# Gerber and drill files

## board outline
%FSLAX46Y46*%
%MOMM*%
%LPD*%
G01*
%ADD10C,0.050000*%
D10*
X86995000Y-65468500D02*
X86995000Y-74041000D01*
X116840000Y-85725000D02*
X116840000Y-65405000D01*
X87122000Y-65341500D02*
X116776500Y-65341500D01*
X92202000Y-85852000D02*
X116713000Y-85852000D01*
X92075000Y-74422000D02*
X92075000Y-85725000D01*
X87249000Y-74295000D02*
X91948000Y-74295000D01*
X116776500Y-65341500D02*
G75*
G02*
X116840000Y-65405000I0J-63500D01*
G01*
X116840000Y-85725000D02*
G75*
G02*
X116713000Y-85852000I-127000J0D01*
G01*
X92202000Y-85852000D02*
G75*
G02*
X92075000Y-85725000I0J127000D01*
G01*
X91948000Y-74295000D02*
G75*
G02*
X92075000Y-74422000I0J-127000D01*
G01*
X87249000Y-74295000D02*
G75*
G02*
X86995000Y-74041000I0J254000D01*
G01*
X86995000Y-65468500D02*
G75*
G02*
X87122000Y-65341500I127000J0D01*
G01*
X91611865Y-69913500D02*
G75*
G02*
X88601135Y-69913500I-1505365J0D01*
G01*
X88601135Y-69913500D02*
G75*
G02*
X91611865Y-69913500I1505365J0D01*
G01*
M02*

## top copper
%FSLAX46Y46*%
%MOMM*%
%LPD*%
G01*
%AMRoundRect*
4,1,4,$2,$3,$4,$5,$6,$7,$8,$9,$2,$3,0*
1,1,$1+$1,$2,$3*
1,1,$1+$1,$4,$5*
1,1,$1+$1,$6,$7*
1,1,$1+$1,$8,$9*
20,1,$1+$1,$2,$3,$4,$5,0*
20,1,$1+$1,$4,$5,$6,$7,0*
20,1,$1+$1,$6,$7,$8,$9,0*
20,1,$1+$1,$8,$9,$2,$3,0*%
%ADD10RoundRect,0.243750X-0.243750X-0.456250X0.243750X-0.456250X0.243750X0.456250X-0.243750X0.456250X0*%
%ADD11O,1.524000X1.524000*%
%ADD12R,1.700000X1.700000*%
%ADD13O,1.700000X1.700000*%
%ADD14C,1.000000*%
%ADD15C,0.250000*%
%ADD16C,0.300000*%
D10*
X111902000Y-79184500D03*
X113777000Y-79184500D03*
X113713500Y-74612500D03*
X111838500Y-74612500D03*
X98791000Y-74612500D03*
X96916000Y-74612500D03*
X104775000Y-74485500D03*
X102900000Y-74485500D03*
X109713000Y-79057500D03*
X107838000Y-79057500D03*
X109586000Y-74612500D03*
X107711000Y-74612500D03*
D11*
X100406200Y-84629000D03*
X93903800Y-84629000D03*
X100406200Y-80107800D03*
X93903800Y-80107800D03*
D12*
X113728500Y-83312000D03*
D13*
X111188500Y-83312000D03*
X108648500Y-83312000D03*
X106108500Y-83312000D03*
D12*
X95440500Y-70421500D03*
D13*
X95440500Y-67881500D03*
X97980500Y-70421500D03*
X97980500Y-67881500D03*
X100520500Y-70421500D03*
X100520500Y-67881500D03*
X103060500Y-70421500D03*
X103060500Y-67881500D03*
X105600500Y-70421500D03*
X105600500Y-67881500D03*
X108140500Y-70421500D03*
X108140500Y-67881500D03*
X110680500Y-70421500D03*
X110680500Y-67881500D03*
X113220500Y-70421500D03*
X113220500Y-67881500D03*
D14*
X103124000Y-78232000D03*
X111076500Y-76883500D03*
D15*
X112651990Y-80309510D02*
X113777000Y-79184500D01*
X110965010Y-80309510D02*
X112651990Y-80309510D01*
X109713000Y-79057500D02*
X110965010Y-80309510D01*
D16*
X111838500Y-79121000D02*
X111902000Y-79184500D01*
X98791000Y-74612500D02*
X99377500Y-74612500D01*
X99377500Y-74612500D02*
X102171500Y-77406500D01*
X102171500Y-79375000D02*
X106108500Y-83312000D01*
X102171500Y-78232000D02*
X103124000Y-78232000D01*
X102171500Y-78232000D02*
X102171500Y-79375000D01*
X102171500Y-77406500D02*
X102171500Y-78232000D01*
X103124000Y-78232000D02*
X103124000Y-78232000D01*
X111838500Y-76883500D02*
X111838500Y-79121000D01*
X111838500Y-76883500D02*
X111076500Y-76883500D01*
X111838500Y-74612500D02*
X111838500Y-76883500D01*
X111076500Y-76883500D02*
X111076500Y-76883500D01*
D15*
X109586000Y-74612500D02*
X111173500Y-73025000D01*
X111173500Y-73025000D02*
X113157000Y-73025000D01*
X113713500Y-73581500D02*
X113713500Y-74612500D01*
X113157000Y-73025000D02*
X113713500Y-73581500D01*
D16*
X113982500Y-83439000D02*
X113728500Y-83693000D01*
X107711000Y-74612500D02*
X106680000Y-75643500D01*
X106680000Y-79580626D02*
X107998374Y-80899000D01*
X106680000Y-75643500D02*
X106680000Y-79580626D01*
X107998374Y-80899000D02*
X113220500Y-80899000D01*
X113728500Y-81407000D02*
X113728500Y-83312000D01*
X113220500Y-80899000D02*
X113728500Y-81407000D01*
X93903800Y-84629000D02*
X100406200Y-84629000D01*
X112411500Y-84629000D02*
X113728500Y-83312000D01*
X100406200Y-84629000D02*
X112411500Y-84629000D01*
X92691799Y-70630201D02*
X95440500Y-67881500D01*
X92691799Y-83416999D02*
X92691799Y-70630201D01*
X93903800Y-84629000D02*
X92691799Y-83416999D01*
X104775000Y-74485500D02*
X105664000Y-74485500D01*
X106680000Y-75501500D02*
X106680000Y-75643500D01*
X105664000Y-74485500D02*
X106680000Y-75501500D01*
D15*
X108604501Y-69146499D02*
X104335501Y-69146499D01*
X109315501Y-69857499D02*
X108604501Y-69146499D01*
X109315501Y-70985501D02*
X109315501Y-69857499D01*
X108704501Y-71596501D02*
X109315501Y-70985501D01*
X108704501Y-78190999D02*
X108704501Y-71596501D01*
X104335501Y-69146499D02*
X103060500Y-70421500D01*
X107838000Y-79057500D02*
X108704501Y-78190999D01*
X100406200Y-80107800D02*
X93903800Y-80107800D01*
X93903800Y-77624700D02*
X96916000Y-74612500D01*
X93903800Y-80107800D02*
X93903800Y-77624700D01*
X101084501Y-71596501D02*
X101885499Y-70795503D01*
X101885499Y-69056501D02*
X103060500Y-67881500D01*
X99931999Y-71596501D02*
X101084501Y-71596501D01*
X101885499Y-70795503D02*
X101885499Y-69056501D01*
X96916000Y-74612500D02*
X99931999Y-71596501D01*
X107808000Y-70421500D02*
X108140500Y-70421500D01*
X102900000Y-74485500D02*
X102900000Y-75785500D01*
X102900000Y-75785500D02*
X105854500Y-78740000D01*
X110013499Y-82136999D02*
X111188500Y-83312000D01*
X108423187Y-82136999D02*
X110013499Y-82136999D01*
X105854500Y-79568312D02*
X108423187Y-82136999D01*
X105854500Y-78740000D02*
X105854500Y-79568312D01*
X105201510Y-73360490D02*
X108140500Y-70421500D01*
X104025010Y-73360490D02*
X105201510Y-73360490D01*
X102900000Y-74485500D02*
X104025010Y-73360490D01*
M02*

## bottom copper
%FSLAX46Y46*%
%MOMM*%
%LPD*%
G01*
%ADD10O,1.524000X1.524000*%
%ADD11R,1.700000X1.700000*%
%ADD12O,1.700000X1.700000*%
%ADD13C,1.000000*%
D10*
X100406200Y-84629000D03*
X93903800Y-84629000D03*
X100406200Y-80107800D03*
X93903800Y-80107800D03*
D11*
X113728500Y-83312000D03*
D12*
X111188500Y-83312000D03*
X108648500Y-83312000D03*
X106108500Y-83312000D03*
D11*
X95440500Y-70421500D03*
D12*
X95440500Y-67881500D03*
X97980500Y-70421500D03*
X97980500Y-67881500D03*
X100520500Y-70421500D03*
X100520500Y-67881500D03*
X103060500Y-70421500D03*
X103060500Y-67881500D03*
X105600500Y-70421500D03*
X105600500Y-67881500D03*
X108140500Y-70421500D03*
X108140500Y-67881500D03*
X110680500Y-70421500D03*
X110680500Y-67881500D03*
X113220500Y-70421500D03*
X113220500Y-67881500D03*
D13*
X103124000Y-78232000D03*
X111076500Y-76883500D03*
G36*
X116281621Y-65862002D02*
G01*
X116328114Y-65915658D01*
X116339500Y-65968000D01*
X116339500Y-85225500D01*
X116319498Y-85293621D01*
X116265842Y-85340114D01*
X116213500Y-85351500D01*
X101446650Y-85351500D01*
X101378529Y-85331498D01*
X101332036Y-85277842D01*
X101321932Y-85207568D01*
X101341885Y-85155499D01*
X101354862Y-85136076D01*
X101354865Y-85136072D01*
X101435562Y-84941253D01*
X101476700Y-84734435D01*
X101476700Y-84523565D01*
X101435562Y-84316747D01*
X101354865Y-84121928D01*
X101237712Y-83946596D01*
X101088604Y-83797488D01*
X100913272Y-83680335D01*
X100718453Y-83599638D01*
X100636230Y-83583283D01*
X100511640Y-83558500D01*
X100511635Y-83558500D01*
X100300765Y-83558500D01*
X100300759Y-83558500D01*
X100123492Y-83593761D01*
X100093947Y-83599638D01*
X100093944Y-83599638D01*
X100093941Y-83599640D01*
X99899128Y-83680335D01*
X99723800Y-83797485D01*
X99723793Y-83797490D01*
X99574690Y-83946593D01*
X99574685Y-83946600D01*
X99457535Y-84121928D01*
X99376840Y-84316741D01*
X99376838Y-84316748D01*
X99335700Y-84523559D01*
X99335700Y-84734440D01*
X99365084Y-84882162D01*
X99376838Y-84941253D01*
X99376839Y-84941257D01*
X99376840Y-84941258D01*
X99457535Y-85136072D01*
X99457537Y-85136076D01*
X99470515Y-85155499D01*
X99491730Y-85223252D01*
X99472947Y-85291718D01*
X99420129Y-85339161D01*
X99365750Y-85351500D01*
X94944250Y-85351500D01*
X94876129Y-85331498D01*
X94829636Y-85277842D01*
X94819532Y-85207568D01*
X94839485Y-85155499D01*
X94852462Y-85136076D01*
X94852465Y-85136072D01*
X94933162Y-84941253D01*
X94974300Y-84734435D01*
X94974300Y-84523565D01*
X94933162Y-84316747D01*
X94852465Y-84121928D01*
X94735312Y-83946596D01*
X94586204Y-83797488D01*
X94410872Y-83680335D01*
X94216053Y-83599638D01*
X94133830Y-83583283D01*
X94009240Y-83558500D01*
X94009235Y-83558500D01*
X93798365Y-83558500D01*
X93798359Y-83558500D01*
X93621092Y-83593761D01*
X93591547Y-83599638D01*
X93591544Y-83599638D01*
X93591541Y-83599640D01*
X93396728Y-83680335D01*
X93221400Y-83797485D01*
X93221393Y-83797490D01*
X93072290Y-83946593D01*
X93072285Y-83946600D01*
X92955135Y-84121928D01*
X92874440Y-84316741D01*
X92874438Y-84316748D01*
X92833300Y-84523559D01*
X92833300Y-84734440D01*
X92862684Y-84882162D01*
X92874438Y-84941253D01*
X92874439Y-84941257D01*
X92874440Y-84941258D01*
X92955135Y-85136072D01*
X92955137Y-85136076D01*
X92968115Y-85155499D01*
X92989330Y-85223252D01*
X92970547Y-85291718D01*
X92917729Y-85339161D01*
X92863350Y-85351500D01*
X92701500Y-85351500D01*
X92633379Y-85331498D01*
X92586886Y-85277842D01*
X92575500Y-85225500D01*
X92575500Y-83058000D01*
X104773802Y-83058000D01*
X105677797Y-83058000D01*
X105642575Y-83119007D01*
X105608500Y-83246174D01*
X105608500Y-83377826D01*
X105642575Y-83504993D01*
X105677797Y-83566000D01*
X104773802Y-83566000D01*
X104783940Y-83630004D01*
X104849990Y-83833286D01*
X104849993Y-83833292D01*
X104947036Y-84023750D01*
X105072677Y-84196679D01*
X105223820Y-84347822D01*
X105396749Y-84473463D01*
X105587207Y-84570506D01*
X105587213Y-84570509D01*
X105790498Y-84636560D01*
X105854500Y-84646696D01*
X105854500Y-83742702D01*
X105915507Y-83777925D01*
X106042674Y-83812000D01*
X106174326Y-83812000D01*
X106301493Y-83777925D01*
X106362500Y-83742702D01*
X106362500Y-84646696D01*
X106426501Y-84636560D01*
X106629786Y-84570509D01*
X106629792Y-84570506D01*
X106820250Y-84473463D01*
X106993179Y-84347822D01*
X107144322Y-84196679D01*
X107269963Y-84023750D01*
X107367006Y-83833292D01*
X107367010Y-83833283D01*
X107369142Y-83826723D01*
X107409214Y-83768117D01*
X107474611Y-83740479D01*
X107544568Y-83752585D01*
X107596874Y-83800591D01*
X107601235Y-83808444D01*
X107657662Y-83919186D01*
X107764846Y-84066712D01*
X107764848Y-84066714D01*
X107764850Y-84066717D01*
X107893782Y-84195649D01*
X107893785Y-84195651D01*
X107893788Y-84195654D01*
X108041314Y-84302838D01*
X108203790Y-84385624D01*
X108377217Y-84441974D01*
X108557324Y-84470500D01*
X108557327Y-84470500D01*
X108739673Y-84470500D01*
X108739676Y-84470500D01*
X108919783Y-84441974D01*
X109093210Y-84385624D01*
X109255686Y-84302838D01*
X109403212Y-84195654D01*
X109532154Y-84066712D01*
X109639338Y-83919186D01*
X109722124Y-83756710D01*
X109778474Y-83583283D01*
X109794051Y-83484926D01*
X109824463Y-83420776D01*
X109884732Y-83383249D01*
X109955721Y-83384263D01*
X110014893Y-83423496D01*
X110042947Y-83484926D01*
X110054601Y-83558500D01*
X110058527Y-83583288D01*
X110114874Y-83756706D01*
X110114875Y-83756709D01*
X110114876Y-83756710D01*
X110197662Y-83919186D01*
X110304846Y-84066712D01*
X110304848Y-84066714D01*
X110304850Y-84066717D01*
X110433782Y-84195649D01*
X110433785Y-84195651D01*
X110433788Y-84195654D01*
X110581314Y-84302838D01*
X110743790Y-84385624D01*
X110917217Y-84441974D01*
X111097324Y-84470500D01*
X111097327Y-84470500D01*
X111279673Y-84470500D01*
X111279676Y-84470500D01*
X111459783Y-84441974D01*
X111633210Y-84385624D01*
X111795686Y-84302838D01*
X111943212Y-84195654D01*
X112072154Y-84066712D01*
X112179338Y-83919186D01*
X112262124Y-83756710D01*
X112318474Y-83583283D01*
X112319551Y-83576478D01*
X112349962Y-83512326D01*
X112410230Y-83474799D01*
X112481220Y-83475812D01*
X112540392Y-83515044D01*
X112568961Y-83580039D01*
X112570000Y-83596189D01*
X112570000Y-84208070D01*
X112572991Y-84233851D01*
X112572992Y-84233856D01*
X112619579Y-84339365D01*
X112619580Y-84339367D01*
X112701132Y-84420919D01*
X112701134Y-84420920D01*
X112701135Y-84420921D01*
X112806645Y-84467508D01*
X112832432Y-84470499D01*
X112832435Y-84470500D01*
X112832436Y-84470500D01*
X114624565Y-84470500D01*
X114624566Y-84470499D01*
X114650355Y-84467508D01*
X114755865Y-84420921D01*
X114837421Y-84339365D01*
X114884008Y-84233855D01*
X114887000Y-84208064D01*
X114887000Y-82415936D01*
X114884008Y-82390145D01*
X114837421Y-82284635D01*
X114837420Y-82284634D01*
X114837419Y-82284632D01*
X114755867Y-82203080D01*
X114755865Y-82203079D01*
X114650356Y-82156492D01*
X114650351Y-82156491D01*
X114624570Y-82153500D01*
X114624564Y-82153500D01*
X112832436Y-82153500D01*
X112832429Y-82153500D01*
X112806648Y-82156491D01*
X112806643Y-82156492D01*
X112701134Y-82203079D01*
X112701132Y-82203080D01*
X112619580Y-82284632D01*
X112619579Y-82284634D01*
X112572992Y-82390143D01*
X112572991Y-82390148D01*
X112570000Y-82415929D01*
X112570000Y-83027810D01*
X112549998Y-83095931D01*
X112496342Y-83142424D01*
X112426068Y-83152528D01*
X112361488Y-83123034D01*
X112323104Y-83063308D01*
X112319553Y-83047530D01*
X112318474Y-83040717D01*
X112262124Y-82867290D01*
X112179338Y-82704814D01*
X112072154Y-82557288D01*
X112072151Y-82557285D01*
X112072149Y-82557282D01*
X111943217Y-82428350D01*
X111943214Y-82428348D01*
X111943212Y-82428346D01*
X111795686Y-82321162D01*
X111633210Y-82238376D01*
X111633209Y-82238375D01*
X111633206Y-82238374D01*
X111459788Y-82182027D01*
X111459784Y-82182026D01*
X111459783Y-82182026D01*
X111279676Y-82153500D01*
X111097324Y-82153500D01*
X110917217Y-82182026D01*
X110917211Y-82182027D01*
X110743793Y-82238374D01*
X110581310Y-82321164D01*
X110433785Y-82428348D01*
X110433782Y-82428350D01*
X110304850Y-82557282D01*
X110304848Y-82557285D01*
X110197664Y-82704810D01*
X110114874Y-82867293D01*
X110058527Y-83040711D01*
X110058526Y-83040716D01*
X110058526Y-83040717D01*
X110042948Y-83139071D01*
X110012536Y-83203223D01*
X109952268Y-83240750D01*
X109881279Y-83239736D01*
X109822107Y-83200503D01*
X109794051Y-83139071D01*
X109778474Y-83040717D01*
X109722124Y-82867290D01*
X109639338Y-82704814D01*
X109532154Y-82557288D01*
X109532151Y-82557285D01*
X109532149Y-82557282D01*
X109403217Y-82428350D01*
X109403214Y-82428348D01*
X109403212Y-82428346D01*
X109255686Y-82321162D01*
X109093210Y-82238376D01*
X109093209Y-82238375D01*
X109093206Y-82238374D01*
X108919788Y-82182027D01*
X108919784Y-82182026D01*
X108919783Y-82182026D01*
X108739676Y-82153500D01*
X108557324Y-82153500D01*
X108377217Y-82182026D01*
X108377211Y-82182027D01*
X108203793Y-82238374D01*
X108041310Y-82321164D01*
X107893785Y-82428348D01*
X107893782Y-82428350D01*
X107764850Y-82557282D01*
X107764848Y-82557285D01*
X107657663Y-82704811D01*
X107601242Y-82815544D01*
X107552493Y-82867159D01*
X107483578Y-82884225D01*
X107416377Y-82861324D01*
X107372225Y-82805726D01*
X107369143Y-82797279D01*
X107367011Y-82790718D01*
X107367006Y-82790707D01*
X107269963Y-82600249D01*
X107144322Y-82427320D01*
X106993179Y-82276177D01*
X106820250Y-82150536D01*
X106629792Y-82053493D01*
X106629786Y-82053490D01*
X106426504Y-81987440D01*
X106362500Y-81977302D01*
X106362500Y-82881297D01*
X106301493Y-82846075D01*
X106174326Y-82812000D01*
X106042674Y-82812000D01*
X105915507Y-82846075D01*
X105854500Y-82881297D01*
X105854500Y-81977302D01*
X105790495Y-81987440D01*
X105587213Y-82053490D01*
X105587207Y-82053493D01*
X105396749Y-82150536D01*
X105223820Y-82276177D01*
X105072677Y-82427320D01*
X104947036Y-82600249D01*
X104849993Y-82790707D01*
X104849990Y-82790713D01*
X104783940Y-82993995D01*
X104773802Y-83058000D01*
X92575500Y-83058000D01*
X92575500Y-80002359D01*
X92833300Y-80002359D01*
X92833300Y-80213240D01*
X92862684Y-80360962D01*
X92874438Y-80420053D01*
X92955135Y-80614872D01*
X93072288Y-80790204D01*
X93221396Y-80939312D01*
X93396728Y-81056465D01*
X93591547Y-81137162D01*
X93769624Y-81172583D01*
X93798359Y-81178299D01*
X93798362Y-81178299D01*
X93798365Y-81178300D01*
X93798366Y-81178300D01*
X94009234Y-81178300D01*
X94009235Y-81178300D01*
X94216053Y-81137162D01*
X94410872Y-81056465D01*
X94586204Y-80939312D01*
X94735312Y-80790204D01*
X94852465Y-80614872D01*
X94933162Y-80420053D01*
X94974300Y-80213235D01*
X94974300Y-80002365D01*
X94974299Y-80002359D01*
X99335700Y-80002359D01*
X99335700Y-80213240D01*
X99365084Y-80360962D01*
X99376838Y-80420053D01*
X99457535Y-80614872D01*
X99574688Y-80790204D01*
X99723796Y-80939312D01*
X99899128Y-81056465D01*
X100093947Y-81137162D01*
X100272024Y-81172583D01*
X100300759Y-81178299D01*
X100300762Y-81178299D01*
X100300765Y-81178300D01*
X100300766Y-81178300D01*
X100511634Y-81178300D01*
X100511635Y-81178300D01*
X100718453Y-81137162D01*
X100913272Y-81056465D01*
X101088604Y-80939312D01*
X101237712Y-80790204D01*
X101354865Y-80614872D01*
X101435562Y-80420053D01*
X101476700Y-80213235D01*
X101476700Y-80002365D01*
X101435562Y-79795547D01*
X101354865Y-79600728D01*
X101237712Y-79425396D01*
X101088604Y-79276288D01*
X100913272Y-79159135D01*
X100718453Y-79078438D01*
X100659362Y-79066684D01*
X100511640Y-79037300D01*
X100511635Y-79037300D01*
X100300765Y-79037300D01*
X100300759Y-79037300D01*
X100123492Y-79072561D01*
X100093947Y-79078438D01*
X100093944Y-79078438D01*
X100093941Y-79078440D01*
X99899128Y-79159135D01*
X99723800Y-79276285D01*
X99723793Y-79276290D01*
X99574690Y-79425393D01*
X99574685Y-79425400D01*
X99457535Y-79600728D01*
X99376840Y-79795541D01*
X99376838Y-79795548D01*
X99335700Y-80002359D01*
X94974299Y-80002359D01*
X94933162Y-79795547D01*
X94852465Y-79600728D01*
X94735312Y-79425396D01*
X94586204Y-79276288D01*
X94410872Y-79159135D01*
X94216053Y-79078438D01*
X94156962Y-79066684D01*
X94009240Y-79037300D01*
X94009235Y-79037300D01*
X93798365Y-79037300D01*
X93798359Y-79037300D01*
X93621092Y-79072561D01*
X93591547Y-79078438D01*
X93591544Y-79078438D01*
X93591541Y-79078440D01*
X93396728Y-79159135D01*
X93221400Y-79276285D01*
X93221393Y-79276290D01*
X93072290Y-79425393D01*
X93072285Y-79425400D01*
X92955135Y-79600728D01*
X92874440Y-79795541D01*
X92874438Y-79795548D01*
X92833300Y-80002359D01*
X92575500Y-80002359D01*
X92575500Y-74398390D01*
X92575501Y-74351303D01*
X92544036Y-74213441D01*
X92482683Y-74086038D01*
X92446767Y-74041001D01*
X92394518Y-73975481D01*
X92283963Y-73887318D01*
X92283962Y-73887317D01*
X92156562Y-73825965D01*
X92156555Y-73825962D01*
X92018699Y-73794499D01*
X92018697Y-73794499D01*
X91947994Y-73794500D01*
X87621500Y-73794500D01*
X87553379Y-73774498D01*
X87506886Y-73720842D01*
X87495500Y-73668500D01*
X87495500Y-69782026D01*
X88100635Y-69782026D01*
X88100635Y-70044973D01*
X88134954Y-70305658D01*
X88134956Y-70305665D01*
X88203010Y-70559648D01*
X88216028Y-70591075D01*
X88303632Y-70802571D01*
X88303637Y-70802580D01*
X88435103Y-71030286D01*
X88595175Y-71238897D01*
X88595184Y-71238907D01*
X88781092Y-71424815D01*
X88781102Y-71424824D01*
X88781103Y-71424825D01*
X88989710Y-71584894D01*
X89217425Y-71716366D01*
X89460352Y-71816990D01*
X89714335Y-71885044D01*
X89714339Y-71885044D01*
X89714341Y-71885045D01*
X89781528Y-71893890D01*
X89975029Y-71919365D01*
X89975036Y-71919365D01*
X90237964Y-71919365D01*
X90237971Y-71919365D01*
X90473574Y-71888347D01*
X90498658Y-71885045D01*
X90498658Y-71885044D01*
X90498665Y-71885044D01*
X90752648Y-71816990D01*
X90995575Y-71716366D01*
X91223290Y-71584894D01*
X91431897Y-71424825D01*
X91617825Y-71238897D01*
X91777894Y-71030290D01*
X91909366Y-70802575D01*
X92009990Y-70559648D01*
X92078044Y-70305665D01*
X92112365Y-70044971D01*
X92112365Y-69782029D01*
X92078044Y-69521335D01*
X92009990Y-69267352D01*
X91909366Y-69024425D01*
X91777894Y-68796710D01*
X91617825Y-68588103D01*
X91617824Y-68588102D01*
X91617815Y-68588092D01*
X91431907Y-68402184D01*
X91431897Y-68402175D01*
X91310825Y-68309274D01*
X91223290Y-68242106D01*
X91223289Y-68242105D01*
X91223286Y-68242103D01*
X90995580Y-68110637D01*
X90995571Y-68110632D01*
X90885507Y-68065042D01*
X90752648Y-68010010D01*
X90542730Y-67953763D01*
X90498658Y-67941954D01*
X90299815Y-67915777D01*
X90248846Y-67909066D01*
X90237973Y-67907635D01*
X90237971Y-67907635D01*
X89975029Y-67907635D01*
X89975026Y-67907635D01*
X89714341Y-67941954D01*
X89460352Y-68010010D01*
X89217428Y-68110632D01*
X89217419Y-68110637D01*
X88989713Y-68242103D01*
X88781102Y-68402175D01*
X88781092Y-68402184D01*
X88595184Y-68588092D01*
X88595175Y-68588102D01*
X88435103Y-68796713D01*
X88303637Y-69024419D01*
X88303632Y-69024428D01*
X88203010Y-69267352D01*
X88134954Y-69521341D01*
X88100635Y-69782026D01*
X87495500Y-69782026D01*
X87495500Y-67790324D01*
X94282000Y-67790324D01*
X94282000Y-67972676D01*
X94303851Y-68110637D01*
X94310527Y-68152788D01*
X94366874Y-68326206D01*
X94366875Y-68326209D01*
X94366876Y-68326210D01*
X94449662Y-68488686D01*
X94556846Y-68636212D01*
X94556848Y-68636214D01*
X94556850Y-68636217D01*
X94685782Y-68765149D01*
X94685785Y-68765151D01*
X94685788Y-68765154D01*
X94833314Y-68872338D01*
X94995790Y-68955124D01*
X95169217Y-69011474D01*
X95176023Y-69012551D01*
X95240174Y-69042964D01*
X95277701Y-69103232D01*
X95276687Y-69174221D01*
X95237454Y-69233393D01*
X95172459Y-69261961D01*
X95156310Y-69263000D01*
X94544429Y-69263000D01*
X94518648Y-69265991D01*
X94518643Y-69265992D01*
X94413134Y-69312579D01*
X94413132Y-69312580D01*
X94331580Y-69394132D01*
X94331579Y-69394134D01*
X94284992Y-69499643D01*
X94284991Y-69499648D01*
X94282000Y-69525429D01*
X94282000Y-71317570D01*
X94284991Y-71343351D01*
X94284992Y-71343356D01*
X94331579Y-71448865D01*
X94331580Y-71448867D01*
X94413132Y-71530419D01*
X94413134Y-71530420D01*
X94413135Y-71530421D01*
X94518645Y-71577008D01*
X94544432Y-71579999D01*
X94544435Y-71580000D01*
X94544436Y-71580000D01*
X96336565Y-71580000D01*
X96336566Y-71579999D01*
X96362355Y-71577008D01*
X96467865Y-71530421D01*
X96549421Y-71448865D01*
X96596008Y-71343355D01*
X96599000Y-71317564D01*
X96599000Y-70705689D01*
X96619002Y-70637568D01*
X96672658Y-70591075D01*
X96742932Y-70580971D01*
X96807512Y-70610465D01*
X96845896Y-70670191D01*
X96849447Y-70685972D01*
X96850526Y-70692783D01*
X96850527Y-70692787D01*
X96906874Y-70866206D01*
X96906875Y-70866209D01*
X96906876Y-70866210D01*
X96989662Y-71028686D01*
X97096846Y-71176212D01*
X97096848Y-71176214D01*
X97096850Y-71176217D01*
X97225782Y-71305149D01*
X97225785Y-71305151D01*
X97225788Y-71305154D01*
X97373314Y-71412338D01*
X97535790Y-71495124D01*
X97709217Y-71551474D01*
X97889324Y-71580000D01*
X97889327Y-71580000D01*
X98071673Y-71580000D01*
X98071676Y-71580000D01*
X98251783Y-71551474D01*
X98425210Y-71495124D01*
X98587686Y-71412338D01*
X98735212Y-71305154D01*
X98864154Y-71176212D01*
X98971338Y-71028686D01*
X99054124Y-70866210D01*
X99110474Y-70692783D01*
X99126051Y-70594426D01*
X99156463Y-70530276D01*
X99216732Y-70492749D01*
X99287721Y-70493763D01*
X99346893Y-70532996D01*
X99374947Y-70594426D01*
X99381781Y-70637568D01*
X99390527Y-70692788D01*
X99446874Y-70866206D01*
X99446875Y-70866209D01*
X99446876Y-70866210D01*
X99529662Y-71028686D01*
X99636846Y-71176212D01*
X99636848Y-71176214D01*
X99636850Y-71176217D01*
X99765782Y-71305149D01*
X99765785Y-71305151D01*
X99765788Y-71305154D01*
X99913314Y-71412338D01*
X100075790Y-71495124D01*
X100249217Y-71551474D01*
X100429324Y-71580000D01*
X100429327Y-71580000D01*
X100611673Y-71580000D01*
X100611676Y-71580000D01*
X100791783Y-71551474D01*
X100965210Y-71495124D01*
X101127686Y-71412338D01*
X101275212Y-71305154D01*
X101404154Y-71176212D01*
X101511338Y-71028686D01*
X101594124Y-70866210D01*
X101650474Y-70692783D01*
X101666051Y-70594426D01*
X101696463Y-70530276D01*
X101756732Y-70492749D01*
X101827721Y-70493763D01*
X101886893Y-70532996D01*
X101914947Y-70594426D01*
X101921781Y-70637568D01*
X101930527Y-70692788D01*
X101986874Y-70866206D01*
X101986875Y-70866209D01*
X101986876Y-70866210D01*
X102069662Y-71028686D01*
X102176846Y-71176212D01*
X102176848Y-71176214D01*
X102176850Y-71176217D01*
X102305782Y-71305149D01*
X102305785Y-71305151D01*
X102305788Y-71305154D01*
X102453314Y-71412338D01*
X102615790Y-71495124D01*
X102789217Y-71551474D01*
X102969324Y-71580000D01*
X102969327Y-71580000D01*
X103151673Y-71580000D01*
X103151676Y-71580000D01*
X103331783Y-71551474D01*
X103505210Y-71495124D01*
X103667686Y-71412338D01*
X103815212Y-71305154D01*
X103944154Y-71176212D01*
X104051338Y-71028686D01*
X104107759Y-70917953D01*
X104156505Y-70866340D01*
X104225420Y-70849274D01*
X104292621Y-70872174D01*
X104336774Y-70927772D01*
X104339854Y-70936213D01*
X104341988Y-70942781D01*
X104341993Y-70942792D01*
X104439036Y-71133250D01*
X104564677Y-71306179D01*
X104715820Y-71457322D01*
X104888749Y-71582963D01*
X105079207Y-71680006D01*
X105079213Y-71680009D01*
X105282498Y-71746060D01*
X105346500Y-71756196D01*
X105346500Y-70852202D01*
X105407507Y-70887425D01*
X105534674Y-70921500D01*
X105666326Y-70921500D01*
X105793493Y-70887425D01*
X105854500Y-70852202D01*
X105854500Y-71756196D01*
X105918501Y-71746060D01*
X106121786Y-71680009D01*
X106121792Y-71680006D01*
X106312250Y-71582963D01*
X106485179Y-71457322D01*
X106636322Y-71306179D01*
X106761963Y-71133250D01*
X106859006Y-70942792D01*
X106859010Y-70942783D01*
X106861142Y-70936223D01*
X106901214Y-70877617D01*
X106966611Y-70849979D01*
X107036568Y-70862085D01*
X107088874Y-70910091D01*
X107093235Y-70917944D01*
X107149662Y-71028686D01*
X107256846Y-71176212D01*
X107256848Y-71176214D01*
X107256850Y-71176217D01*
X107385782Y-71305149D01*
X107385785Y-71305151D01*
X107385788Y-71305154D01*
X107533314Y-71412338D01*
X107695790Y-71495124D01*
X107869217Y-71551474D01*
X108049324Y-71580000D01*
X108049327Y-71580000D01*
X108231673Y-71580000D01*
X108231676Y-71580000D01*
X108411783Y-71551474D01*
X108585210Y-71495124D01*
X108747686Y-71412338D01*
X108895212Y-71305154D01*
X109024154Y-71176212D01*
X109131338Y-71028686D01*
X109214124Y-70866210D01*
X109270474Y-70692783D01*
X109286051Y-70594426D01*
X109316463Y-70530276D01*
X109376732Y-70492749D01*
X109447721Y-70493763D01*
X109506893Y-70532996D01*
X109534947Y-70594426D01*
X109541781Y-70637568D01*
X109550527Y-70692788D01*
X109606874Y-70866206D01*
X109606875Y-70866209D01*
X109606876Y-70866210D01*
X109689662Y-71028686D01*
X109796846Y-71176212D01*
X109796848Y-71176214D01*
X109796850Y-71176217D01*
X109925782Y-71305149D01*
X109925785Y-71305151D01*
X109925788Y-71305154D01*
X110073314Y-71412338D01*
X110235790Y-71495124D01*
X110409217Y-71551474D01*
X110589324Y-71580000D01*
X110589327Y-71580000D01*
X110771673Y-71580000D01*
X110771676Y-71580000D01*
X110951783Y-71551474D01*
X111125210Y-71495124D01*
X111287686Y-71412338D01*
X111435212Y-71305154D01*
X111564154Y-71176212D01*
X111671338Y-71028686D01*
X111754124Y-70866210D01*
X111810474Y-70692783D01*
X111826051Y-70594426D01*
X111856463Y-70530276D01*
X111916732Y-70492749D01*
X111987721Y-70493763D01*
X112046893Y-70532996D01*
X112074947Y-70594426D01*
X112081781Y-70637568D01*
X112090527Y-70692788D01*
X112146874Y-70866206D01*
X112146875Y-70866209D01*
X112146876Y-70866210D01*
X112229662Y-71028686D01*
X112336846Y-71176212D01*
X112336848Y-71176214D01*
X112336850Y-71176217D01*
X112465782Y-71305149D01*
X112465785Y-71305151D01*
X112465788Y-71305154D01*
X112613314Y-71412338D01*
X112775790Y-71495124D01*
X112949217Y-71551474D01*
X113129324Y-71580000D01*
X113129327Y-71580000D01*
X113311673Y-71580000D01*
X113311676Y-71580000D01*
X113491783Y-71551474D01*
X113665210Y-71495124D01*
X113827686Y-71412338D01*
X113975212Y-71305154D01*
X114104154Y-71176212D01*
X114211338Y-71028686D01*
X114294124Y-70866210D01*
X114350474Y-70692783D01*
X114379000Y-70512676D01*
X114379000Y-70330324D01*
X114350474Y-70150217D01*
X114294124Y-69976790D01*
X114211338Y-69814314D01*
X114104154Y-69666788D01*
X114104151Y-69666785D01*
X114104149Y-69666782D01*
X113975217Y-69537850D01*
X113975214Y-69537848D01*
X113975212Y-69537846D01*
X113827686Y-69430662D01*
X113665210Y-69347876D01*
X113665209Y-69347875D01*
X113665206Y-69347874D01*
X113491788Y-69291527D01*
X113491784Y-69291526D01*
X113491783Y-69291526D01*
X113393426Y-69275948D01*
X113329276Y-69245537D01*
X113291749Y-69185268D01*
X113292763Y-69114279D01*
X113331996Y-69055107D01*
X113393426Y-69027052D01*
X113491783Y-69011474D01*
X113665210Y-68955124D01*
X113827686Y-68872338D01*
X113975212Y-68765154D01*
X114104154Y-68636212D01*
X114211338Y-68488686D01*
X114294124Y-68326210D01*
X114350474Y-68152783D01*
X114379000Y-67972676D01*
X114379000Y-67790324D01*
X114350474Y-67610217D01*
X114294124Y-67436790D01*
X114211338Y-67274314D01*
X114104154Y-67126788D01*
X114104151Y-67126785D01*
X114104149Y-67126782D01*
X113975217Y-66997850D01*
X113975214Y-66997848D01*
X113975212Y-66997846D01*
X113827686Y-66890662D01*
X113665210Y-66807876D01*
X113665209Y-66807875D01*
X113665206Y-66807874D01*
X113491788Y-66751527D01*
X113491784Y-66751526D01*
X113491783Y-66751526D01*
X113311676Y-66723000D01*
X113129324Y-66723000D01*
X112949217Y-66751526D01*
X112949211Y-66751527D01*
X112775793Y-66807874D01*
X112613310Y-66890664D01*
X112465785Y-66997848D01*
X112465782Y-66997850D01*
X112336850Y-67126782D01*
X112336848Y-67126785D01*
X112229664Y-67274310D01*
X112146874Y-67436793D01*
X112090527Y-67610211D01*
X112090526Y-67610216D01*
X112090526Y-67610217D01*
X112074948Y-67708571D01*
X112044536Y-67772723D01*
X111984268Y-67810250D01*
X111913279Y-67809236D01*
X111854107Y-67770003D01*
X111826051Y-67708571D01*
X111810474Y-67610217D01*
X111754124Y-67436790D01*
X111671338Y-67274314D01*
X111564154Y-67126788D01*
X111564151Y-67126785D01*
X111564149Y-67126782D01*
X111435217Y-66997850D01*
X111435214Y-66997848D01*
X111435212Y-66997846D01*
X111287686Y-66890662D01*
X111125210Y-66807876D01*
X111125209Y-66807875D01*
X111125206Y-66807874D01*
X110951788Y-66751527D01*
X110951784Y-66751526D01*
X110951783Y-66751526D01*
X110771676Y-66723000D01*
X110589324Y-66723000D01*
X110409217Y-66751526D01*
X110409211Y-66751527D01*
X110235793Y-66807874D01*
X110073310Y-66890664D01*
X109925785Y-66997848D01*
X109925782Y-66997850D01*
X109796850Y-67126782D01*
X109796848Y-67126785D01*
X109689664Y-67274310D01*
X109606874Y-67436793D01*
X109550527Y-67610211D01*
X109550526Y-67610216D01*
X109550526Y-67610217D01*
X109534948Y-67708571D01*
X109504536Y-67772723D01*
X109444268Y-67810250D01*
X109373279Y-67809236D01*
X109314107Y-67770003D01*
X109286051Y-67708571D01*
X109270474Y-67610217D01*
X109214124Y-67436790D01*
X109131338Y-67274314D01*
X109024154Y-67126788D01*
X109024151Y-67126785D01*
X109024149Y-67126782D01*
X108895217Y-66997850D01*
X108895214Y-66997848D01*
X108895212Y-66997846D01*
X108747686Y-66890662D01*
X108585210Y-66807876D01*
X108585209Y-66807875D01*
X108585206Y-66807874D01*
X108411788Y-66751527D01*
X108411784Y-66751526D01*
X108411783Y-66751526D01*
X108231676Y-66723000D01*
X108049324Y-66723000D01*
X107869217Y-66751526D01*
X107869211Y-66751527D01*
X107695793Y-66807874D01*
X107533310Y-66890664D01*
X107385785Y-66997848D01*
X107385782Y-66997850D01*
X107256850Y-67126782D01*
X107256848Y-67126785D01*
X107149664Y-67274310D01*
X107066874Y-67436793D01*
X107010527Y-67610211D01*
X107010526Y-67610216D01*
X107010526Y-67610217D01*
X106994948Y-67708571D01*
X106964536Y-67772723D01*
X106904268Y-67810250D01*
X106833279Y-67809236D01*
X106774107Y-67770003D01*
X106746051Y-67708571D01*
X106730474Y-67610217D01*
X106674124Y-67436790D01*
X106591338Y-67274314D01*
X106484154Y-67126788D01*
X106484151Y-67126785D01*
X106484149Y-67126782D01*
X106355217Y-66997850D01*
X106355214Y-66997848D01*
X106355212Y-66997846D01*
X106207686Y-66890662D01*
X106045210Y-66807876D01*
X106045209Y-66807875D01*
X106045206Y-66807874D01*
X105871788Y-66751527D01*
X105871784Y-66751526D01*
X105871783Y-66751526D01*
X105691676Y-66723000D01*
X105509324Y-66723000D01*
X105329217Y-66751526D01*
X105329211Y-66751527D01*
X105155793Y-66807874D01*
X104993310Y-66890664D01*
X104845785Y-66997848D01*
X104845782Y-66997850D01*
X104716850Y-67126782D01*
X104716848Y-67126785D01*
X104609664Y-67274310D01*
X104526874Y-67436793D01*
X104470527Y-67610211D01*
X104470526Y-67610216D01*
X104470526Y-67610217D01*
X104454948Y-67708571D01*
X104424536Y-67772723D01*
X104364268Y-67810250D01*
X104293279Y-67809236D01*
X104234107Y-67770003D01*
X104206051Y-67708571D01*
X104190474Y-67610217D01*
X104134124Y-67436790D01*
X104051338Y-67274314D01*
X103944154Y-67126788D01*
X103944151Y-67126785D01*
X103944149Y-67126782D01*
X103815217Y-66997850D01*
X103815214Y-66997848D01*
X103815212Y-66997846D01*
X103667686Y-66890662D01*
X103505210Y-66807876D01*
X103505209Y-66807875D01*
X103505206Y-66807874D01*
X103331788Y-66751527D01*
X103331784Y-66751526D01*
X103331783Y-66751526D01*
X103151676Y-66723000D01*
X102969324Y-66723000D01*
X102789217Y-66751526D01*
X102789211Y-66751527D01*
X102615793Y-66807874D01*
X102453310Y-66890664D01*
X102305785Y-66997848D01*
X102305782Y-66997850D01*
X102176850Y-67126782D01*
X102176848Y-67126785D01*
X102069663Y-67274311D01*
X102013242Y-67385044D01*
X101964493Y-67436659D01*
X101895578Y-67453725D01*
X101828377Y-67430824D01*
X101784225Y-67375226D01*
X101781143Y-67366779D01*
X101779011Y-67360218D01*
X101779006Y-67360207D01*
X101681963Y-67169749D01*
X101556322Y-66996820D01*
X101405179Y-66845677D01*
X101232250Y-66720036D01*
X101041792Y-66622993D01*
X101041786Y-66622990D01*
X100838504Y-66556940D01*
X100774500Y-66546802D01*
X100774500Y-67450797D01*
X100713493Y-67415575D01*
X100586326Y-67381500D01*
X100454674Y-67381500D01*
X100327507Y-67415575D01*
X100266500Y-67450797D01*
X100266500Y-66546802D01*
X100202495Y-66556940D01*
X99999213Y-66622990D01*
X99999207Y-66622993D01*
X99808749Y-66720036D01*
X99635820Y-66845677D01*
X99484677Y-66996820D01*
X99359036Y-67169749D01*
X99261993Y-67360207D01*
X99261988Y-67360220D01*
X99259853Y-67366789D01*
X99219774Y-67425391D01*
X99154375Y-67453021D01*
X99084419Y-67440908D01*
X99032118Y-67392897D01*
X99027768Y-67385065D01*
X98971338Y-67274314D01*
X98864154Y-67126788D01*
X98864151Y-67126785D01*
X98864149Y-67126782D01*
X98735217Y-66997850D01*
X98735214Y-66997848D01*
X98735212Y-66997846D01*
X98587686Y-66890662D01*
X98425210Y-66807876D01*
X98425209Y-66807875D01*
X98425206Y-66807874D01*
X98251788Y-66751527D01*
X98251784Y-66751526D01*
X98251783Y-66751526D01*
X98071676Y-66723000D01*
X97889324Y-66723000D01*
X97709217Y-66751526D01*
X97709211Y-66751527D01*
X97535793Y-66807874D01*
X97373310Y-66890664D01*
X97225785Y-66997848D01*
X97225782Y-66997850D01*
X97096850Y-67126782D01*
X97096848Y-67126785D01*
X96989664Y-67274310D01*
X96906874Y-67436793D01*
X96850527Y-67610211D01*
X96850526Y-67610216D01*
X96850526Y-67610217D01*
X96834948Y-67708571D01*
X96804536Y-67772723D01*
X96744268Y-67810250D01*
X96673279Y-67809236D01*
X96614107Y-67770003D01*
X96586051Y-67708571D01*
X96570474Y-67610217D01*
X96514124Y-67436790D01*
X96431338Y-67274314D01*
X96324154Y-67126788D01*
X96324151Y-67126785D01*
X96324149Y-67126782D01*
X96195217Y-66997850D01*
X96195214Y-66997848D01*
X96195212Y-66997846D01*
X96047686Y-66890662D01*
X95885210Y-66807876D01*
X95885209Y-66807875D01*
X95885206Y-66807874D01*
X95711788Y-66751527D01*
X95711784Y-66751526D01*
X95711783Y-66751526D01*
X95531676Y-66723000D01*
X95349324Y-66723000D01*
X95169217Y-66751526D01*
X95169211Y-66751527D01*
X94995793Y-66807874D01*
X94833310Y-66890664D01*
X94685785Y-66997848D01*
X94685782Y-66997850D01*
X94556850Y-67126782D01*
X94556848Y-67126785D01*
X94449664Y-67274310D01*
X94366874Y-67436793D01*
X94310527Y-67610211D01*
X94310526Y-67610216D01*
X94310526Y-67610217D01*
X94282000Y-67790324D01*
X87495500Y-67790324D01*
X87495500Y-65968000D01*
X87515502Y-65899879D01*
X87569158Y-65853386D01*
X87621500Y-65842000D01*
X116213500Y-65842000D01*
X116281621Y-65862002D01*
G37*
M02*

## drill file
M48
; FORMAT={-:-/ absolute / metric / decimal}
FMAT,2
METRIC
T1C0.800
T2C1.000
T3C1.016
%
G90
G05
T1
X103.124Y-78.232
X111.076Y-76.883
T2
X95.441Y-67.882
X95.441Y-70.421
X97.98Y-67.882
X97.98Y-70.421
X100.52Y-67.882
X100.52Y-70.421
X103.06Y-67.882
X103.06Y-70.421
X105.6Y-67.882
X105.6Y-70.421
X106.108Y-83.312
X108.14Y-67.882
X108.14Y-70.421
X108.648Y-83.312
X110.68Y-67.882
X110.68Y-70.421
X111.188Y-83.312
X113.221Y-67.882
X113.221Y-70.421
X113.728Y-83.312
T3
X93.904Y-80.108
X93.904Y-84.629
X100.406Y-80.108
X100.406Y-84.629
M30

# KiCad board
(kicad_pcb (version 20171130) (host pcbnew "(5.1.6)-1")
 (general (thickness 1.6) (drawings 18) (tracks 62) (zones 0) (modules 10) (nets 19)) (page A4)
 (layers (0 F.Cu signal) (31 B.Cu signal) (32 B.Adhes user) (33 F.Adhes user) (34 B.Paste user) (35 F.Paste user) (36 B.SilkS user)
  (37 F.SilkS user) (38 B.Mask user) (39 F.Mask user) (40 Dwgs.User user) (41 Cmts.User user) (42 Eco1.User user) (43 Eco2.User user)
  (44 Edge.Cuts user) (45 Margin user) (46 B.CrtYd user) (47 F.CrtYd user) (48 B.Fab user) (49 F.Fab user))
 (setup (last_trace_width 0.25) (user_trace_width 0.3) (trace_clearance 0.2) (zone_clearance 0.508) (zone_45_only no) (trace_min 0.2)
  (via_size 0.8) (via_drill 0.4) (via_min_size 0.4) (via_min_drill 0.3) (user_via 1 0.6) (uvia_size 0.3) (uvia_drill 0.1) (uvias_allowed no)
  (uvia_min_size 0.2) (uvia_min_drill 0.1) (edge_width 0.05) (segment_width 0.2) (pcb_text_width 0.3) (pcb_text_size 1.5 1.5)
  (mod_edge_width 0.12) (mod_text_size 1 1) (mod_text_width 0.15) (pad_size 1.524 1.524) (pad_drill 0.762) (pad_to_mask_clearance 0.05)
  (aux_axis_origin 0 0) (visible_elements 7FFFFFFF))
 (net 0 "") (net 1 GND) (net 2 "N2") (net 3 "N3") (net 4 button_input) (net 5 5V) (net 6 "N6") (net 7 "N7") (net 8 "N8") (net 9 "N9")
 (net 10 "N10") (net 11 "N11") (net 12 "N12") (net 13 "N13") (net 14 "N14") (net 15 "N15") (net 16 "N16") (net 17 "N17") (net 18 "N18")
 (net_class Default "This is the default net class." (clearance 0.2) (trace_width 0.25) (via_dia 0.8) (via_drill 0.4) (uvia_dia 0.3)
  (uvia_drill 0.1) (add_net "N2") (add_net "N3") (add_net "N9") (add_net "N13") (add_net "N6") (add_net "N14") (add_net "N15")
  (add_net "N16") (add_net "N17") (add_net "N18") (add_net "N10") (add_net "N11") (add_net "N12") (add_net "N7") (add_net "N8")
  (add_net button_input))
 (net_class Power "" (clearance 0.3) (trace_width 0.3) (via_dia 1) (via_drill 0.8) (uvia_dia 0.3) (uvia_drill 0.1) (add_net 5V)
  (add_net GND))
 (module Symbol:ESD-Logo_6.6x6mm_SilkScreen (layer B.Cu) (at 98.171 75.438 180)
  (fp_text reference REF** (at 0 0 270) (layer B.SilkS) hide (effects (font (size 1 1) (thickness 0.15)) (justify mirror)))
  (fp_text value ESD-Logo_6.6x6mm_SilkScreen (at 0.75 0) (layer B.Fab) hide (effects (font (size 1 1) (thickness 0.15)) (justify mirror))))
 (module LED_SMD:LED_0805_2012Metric (layer F.Cu) (at 112.8395 79.1845)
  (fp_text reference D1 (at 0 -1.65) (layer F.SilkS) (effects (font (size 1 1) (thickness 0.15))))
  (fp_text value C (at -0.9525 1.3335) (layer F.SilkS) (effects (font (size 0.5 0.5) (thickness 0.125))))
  (pad 1 smd roundrect (at -0.9375 0) (size 0.975 1.4) (layers F.Cu F.Paste F.Mask) (roundrect_rratio 0.25) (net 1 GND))
  (pad 2 smd roundrect (at 0.9375 0) (size 0.975 1.4) (layers F.Cu F.Paste F.Mask) (roundrect_rratio 0.25) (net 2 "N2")))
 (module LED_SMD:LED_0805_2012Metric (layer F.Cu) (at 112.776 74.6125)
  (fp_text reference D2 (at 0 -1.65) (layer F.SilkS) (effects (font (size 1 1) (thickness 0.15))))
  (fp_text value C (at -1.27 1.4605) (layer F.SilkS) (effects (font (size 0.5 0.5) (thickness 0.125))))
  (pad 2 smd roundrect (at 0.9375 0) (size 0.975 1.4) (layers F.Cu F.Paste F.Mask) (roundrect_rratio 0.25) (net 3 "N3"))
  (pad 1 smd roundrect (at -0.9375 0) (size 0.975 1.4) (layers F.Cu F.Paste F.Mask) (roundrect_rratio 0.25) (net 1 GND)))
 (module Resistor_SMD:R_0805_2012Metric (layer F.Cu) (at 97.8535 74.6125)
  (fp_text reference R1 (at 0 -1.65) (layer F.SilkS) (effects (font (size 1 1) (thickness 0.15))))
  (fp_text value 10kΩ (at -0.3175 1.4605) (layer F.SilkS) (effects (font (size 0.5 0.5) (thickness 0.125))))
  (pad 2 smd roundrect (at 0.9375 0) (size 0.975 1.4) (layers F.Cu F.Paste F.Mask) (roundrect_rratio 0.25) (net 1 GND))
  (pad 1 smd roundrect (at -0.9375 0) (size 0.975 1.4) (layers F.Cu F.Paste F.Mask) (roundrect_rratio 0.25) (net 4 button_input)))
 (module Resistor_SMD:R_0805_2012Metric (layer F.Cu) (at 103.8375 74.4855)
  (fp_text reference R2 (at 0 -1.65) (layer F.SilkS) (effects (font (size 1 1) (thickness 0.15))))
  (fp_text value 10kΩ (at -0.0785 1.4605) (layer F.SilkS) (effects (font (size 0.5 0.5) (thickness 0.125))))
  (pad 2 smd roundrect (at 0.9375 0) (size 0.975 1.4) (layers F.Cu F.Paste F.Mask) (roundrect_rratio 0.25) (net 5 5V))
  (pad 1 smd roundrect (at -0.9375 0) (size 0.975 1.4) (layers F.Cu F.Paste F.Mask) (roundrect_rratio 0.25) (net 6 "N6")))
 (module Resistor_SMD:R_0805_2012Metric (layer F.Cu) (at 108.7755 79.0575)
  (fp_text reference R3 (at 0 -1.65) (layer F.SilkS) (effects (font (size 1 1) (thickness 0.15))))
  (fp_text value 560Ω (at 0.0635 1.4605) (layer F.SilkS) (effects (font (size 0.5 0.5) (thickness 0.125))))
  (pad 2 smd roundrect (at 0.9375 0) (size 0.975 1.4) (layers F.Cu F.Paste F.Mask) (roundrect_rratio 0.25) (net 2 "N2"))
  (pad 1 smd roundrect (at -0.9375 0) (size 0.975 1.4) (layers F.Cu F.Paste F.Mask) (roundrect_rratio 0.25) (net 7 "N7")))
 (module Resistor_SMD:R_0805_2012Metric (layer F.Cu) (at 108.6485 74.6125)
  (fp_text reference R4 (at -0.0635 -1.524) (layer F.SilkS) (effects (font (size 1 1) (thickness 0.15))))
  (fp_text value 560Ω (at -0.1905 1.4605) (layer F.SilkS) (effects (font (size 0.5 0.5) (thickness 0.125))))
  (pad 2 smd roundrect (at 0.9375 0) (size 0.975 1.4) (layers F.Cu F.Paste F.Mask) (roundrect_rratio 0.25) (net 3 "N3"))
  (pad 1 smd roundrect (at -0.9375 0) (size 0.975 1.4) (layers F.Cu F.Paste F.Mask) (roundrect_rratio 0.25) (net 5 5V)))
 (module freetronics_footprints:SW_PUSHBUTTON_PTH (layer F.Cu) (at 97.155 82.3684 180)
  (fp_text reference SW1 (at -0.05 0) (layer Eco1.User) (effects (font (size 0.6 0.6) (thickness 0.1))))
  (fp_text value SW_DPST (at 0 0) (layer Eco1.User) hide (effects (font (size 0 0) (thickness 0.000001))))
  (pad 1 thru_hole oval (at -3.2512 -2.2606 180) (size 1.524 1.524) (drill 1.016) (layers *.Cu *.Mask) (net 5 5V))
  (pad 1 thru_hole oval (at 3.2512 -2.2606 180) (size 1.524 1.524) (drill 1.016) (layers *.Cu *.Mask) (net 5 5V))
  (pad 2 thru_hole oval (at -3.2512 2.2606 180) (size 1.524 1.524) (drill 1.016) (layers *.Cu *.Mask) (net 4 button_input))
  (pad 2 thru_hole oval (at 3.2512 2.2606 180) (size 1.524 1.524) (drill 1.016) (layers *.Cu *.Mask) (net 4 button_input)))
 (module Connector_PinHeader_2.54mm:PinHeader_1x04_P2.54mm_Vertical (layer F.Cu) (at 113.7285 83.312 270)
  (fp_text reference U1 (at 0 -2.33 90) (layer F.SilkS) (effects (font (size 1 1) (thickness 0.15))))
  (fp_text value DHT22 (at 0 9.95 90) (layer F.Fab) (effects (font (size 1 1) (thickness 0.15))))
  (pad 1 thru_hole rect (at 0 0 270) (size 1.7 1.7) (drill 1) (layers *.Cu *.Mask) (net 5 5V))
  (pad 2 thru_hole oval (at 0 2.54 270) (size 1.7 1.7) (drill 1) (layers *.Cu *.Mask) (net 6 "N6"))
  (pad 3 thru_hole oval (at 0 5.08 270) (size 1.7 1.7) (drill 1) (layers *.Cu *.Mask) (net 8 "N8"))
  (pad 4 thru_hole oval (at 0 7.62 270) (size 1.7 1.7) (drill 1) (layers *.Cu *.Mask) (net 1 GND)))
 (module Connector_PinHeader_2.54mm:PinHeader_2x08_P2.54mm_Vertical (layer F.Cu) (at 95.4405 70.4215 90)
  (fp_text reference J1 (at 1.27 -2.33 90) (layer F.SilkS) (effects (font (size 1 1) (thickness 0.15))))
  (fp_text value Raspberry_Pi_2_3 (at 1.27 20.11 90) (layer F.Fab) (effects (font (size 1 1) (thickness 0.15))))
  (pad 1 thru_hole rect (at 0 0 90) (size 1.7 1.7) (drill 1) (layers *.Cu *.Mask) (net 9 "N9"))
  (pad 2 thru_hole oval (at 2.54 0 90) (size 1.7 1.7) (drill 1) (layers *.Cu *.Mask) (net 5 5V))
  (pad 3 thru_hole oval (at 0 2.54 90) (size 1.7 1.7) (drill 1) (layers *.Cu *.Mask) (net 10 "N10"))
  (pad 4 thru_hole oval (at 2.54 2.54 90) (size 1.7 1.7) (drill 1) (layers *.Cu *.Mask) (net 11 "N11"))
  (pad 5 thru_hole oval (at 0 5.08 90) (size 1.7 1.7) (drill 1) (layers *.Cu *.Mask) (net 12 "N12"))
  (pad 6 thru_hole oval (at 2.54 5.08 90) (size 1.7 1.7) (drill 1) (layers *.Cu *.Mask) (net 1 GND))
  (pad 7 thru_hole oval (at 0 7.62 90) (size 1.7 1.7) (drill 1) (layers *.Cu *.Mask) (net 7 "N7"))
  (pad 8 thru_hole oval (at 2.54 7.62 90) (size 1.7 1.7) (drill 1) (layers *.Cu *.Mask) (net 4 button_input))
  (pad 9 thru_hole oval (at 0 10.16 90) (size 1.7 1.7) (drill 1) (layers *.Cu *.Mask) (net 1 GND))
  (pad 10 thru_hole oval (at 2.54 10.16 90) (size 1.7 1.7) (drill 1) (layers *.Cu *.Mask) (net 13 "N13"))
  (pad 11 thru_hole oval (at 0 12.7 90) (size 1.7 1.7) (drill 1) (layers *.Cu *.Mask) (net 6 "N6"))
  (pad 12 thru_hole oval (at 2.54 12.7 90) (size 1.7 1.7) (drill 1) (layers *.Cu *.Mask) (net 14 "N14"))
  (pad 13 thru_hole oval (at 0 15.24 90) (size 1.7 1.7) (drill 1) (layers *.Cu *.Mask) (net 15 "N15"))
  (pad 14 thru_hole oval (at 2.54 15.24 90) (size 1.7 1.7) (drill 1) (layers *.Cu *.Mask) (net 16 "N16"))
  (pad 15 thru_hole oval (at 0 17.78 90) (size 1.7 1.7) (drill 1) (layers *.Cu *.Mask) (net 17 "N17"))
  (pad 16 thru_hole oval (at 2.54 17.78 90) (size 1.7 1.7) (drill 1) (layers *.Cu *.Mask) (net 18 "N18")))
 (gr_line (start 86.995 65.4685) (end 86.995 74.041) (layer Edge.Cuts) (width 0.05))
 (gr_line (start 116.84 85.725) (end 116.84 65.405) (layer Edge.Cuts) (width 0.05))
 (gr_line (start 87.122 65.3415) (end 116.7765 65.3415) (layer Edge.Cuts) (width 0.05))
 (gr_line (start 92.202 85.852) (end 116.713 85.852) (layer Edge.Cuts) (width 0.05))
 (gr_line (start 92.075 74.422) (end 92.075 85.725) (layer Edge.Cuts) (width 0.05))
 (gr_line (start 87.249 74.295) (end 91.948 74.295) (layer Edge.Cuts) (width 0.05))
 (gr_arc (start 116.7765 65.405) (end 116.84 65.405) (angle -90) (layer Edge.Cuts) (width 0.05))
 (gr_arc (start 116.713 85.725) (end 116.713 85.852) (angle -90) (layer Edge.Cuts) (width 0.05))
 (gr_arc (start 92.202 85.725) (end 92.075 85.725) (angle -90) (layer Edge.Cuts) (width 0.05))
 (gr_arc (start 91.948 74.422) (end 92.075 74.422) (angle -90) (layer Edge.Cuts) (width 0.05))
 (gr_arc (start 87.249 74.041) (end 86.995 74.041) (angle -90) (layer Edge.Cuts) (width 0.05))
 (gr_arc (start 87.122 65.4685) (end 87.122 65.3415) (angle -90) (layer Edge.Cuts) (width 0.05))
 (gr_circle (center 90.1065 69.9135) (end 90.805 71.247) (layer Edge.Cuts) (width 0.05))
 (segment (start 112.65199 80.30951) (end 113.777 79.1845) (width 0.25) (layer F.Cu) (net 2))
 (segment (start 110.96501 80.30951) (end 112.65199 80.30951) (width 0.25) (layer F.Cu) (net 2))
 (segment (start 109.713 79.0575) (end 110.96501 80.30951) (width 0.25) (layer F.Cu) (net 2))
 (segment (start 111.8385 79.121) (end 111.902 79.1845) (width 0.3) (layer F.Cu) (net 1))
 (segment (start 98.791 74.6125) (end 99.3775 74.6125) (width 0.3) (layer F.Cu) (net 1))
 (segment (start 99.3775 74.6125) (end 102.1715 77.4065) (width 0.3) (layer F.Cu) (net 1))
 (segment (start 102.1715 79.375) (end 106.1085 83.312) (width 0.3) (layer F.Cu) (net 1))
 (segment (start 102.1715 78.232) (end 103.124 78.232) (width 0.3) (layer F.Cu) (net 1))
 (segment (start 102.1715 78.232) (end 102.1715 79.375) (width 0.3) (layer F.Cu) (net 1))
 (segment (start 102.1715 77.4065) (end 102.1715 78.232) (width 0.3) (layer F.Cu) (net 1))
 (segment (start 103.124 78.232) (end 103.124 78.232) (width 0.3) (layer F.Cu) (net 1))
 (via (at 103.124 78.232) (size 1) (drill 0.8) (layers F.Cu B.Cu) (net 1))
 (segment (start 111.8385 76.8835) (end 111.8385 79.121) (width 0.3) (layer F.Cu) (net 1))
 (segment (start 111.8385 76.8835) (end 111.0765 76.8835) (width 0.3) (layer F.Cu) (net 1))
 (segment (start 111.8385 74.6125) (end 111.8385 76.8835) (width 0.3) (layer F.Cu) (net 1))
 (segment (start 111.0765 76.8835) (end 111.0765 76.8835) (width 0.3) (layer F.Cu) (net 1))
 (via (at 111.0765 76.8835) (size 1) (drill 0.8) (layers F.Cu B.Cu) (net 1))
 (segment (start 109.586 74.6125) (end 111.1735 73.025) (width 0.25) (layer F.Cu) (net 3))
 (segment (start 111.1735 73.025) (end 113.157 73.025) (width 0.25) (layer F.Cu) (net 3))
 (segment (start 113.7135 73.5815) (end 113.7135 74.6125) (width 0.25) (layer F.Cu) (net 3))
 (segment (start 113.157 73.025) (end 113.7135 73.5815) (width 0.25) (layer F.Cu) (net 3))
 (segment (start 113.9825 83.439) (end 113.7285 83.693) (width 0.3) (layer F.Cu) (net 5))
 (segment (start 107.711 74.6125) (end 106.68 75.6435) (width 0.3) (layer F.Cu) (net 5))
 (segment (start 106.68 79.580626) (end 107.998374 80.899) (width 0.3) (layer F.Cu) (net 5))
 (segment (start 106.68 75.6435) (end 106.68 79.580626) (width 0.3) (layer F.Cu) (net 5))
 (segment (start 107.998374 80.899) (end 113.2205 80.899) (width 0.3) (layer F.Cu) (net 5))
 (segment (start 113.7285 81.407) (end 113.7285 83.312) (width 0.3) (layer F.Cu) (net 5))
 (segment (start 113.2205 80.899) (end 113.7285 81.407) (width 0.3) (layer F.Cu) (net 5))
 (segment (start 93.9038 84.629) (end 100.4062 84.629) (width 0.3) (layer F.Cu) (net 5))
 (segment (start 112.4115 84.629) (end 113.7285 83.312) (width 0.3) (layer F.Cu) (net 5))
 (segment (start 100.4062 84.629) (end 112.4115 84.629) (width 0.3) (layer F.Cu) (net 5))
 (segment (start 92.691799 70.630201) (end 95.4405 67.8815) (width 0.3) (layer F.Cu) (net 5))
 (segment (start 92.691799 83.416999) (end 92.691799 70.630201) (width 0.3) (layer F.Cu) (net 5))
 (segment (start 93.9038 84.629) (end 92.691799 83.416999) (width 0.3) (layer F.Cu) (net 5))
 (segment (start 104.775 74.4855) (end 105.664 74.4855) (width 0.3) (layer F.Cu) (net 5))
 (segment (start 106.68 75.5015) (end 106.68 75.6435) (width 0.3) (layer F.Cu) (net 5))
 (segment (start 105.664 74.4855) (end 106.68 75.5015) (width 0.3) (layer F.Cu) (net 5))
 (segment (start 108.604501 69.146499) (end 104.335501 69.146499) (width 0.25) (layer F.Cu) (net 7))
 (segment (start 109.315501 69.857499) (end 108.604501 69.146499) (width 0.25) (layer F.Cu) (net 7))
 (segment (start 109.315501 70.985501) (end 109.315501 69.857499) (width 0.25) (layer F.Cu) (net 7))
 (segment (start 108.704501 71.596501) (end 109.315501 70.985501) (width 0.25) (layer F.Cu) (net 7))
 (segment (start 108.704501 78.190999) (end 108.704501 71.596501) (width 0.25) (layer F.Cu) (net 7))
 (segment (start 104.335501 69.146499) (end 103.0605 70.4215) (width 0.25) (layer F.Cu) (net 7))
 (segment (start 107.838 79.0575) (end 108.704501 78.190999) (width 0.25) (layer F.Cu) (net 7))
 (segment (start 100.4062 80.1078) (end 93.9038 80.1078) (width 0.25) (layer F.Cu) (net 4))
 (segment (start 93.9038 77.6247) (end 96.916 74.6125) (width 0.25) (layer F.Cu) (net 4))
 (segment (start 93.9038 80.1078) (end 93.9038 77.6247) (width 0.25) (layer F.Cu) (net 4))
 (segment (start 101.084501 71.596501) (end 101.885499 70.795503) (width 0.25) (layer F.Cu) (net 4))
 (segment (start 101.885499 69.056501) (end 103.0605 67.8815) (width 0.25) (layer F.Cu) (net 4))
 (segment (start 99.931999 71.596501) (end 101.084501 71.596501) (width 0.25) (layer F.Cu) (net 4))
 (segment (start 101.885499 70.795503) (end 101.885499 69.056501) (width 0.25) (layer F.Cu) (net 4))
 (segment (start 96.916 74.6125) (end 99.931999 71.596501) (width 0.25) (layer F.Cu) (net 4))
 (segment (start 107.808 70.4215) (end 108.1405 70.4215) (width 0.25) (layer F.Cu) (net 6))
 (segment (start 102.9 74.4855) (end 102.9 75.7855) (width 0.25) (layer F.Cu) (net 6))
 (segment (start 102.9 75.7855) (end 105.8545 78.74) (width 0.25) (layer F.Cu) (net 6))
 (segment (start 110.013499 82.136999) (end 111.1885 83.312) (width 0.25) (layer F.Cu) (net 6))
 (segment (start 108.423187 82.136999) (end 110.013499 82.136999) (width 0.25) (layer F.Cu) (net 6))
 (segment (start 105.8545 79.568312) (end 108.423187 82.136999) (width 0.25) (layer F.Cu) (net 6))
 (segment (start 105.8545 78.74) (end 105.8545 79.568312) (width 0.25) (layer F.Cu) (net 6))
 (segment (start 105.20151 73.36049) (end 108.1405 70.4215) (width 0.25) (layer F.Cu) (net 6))
 (segment (start 104.02501 73.36049) (end 105.20151 73.36049) (width 0.25) (layer F.Cu) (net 6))
 (segment (start 102.9 74.4855) (end 104.02501 73.36049) (width 0.25) (layer F.Cu) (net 6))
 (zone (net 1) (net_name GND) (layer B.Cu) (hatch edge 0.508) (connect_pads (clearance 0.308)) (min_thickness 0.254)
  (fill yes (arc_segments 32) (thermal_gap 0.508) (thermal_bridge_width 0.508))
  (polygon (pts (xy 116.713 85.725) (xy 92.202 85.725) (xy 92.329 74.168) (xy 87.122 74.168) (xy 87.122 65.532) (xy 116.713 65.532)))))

